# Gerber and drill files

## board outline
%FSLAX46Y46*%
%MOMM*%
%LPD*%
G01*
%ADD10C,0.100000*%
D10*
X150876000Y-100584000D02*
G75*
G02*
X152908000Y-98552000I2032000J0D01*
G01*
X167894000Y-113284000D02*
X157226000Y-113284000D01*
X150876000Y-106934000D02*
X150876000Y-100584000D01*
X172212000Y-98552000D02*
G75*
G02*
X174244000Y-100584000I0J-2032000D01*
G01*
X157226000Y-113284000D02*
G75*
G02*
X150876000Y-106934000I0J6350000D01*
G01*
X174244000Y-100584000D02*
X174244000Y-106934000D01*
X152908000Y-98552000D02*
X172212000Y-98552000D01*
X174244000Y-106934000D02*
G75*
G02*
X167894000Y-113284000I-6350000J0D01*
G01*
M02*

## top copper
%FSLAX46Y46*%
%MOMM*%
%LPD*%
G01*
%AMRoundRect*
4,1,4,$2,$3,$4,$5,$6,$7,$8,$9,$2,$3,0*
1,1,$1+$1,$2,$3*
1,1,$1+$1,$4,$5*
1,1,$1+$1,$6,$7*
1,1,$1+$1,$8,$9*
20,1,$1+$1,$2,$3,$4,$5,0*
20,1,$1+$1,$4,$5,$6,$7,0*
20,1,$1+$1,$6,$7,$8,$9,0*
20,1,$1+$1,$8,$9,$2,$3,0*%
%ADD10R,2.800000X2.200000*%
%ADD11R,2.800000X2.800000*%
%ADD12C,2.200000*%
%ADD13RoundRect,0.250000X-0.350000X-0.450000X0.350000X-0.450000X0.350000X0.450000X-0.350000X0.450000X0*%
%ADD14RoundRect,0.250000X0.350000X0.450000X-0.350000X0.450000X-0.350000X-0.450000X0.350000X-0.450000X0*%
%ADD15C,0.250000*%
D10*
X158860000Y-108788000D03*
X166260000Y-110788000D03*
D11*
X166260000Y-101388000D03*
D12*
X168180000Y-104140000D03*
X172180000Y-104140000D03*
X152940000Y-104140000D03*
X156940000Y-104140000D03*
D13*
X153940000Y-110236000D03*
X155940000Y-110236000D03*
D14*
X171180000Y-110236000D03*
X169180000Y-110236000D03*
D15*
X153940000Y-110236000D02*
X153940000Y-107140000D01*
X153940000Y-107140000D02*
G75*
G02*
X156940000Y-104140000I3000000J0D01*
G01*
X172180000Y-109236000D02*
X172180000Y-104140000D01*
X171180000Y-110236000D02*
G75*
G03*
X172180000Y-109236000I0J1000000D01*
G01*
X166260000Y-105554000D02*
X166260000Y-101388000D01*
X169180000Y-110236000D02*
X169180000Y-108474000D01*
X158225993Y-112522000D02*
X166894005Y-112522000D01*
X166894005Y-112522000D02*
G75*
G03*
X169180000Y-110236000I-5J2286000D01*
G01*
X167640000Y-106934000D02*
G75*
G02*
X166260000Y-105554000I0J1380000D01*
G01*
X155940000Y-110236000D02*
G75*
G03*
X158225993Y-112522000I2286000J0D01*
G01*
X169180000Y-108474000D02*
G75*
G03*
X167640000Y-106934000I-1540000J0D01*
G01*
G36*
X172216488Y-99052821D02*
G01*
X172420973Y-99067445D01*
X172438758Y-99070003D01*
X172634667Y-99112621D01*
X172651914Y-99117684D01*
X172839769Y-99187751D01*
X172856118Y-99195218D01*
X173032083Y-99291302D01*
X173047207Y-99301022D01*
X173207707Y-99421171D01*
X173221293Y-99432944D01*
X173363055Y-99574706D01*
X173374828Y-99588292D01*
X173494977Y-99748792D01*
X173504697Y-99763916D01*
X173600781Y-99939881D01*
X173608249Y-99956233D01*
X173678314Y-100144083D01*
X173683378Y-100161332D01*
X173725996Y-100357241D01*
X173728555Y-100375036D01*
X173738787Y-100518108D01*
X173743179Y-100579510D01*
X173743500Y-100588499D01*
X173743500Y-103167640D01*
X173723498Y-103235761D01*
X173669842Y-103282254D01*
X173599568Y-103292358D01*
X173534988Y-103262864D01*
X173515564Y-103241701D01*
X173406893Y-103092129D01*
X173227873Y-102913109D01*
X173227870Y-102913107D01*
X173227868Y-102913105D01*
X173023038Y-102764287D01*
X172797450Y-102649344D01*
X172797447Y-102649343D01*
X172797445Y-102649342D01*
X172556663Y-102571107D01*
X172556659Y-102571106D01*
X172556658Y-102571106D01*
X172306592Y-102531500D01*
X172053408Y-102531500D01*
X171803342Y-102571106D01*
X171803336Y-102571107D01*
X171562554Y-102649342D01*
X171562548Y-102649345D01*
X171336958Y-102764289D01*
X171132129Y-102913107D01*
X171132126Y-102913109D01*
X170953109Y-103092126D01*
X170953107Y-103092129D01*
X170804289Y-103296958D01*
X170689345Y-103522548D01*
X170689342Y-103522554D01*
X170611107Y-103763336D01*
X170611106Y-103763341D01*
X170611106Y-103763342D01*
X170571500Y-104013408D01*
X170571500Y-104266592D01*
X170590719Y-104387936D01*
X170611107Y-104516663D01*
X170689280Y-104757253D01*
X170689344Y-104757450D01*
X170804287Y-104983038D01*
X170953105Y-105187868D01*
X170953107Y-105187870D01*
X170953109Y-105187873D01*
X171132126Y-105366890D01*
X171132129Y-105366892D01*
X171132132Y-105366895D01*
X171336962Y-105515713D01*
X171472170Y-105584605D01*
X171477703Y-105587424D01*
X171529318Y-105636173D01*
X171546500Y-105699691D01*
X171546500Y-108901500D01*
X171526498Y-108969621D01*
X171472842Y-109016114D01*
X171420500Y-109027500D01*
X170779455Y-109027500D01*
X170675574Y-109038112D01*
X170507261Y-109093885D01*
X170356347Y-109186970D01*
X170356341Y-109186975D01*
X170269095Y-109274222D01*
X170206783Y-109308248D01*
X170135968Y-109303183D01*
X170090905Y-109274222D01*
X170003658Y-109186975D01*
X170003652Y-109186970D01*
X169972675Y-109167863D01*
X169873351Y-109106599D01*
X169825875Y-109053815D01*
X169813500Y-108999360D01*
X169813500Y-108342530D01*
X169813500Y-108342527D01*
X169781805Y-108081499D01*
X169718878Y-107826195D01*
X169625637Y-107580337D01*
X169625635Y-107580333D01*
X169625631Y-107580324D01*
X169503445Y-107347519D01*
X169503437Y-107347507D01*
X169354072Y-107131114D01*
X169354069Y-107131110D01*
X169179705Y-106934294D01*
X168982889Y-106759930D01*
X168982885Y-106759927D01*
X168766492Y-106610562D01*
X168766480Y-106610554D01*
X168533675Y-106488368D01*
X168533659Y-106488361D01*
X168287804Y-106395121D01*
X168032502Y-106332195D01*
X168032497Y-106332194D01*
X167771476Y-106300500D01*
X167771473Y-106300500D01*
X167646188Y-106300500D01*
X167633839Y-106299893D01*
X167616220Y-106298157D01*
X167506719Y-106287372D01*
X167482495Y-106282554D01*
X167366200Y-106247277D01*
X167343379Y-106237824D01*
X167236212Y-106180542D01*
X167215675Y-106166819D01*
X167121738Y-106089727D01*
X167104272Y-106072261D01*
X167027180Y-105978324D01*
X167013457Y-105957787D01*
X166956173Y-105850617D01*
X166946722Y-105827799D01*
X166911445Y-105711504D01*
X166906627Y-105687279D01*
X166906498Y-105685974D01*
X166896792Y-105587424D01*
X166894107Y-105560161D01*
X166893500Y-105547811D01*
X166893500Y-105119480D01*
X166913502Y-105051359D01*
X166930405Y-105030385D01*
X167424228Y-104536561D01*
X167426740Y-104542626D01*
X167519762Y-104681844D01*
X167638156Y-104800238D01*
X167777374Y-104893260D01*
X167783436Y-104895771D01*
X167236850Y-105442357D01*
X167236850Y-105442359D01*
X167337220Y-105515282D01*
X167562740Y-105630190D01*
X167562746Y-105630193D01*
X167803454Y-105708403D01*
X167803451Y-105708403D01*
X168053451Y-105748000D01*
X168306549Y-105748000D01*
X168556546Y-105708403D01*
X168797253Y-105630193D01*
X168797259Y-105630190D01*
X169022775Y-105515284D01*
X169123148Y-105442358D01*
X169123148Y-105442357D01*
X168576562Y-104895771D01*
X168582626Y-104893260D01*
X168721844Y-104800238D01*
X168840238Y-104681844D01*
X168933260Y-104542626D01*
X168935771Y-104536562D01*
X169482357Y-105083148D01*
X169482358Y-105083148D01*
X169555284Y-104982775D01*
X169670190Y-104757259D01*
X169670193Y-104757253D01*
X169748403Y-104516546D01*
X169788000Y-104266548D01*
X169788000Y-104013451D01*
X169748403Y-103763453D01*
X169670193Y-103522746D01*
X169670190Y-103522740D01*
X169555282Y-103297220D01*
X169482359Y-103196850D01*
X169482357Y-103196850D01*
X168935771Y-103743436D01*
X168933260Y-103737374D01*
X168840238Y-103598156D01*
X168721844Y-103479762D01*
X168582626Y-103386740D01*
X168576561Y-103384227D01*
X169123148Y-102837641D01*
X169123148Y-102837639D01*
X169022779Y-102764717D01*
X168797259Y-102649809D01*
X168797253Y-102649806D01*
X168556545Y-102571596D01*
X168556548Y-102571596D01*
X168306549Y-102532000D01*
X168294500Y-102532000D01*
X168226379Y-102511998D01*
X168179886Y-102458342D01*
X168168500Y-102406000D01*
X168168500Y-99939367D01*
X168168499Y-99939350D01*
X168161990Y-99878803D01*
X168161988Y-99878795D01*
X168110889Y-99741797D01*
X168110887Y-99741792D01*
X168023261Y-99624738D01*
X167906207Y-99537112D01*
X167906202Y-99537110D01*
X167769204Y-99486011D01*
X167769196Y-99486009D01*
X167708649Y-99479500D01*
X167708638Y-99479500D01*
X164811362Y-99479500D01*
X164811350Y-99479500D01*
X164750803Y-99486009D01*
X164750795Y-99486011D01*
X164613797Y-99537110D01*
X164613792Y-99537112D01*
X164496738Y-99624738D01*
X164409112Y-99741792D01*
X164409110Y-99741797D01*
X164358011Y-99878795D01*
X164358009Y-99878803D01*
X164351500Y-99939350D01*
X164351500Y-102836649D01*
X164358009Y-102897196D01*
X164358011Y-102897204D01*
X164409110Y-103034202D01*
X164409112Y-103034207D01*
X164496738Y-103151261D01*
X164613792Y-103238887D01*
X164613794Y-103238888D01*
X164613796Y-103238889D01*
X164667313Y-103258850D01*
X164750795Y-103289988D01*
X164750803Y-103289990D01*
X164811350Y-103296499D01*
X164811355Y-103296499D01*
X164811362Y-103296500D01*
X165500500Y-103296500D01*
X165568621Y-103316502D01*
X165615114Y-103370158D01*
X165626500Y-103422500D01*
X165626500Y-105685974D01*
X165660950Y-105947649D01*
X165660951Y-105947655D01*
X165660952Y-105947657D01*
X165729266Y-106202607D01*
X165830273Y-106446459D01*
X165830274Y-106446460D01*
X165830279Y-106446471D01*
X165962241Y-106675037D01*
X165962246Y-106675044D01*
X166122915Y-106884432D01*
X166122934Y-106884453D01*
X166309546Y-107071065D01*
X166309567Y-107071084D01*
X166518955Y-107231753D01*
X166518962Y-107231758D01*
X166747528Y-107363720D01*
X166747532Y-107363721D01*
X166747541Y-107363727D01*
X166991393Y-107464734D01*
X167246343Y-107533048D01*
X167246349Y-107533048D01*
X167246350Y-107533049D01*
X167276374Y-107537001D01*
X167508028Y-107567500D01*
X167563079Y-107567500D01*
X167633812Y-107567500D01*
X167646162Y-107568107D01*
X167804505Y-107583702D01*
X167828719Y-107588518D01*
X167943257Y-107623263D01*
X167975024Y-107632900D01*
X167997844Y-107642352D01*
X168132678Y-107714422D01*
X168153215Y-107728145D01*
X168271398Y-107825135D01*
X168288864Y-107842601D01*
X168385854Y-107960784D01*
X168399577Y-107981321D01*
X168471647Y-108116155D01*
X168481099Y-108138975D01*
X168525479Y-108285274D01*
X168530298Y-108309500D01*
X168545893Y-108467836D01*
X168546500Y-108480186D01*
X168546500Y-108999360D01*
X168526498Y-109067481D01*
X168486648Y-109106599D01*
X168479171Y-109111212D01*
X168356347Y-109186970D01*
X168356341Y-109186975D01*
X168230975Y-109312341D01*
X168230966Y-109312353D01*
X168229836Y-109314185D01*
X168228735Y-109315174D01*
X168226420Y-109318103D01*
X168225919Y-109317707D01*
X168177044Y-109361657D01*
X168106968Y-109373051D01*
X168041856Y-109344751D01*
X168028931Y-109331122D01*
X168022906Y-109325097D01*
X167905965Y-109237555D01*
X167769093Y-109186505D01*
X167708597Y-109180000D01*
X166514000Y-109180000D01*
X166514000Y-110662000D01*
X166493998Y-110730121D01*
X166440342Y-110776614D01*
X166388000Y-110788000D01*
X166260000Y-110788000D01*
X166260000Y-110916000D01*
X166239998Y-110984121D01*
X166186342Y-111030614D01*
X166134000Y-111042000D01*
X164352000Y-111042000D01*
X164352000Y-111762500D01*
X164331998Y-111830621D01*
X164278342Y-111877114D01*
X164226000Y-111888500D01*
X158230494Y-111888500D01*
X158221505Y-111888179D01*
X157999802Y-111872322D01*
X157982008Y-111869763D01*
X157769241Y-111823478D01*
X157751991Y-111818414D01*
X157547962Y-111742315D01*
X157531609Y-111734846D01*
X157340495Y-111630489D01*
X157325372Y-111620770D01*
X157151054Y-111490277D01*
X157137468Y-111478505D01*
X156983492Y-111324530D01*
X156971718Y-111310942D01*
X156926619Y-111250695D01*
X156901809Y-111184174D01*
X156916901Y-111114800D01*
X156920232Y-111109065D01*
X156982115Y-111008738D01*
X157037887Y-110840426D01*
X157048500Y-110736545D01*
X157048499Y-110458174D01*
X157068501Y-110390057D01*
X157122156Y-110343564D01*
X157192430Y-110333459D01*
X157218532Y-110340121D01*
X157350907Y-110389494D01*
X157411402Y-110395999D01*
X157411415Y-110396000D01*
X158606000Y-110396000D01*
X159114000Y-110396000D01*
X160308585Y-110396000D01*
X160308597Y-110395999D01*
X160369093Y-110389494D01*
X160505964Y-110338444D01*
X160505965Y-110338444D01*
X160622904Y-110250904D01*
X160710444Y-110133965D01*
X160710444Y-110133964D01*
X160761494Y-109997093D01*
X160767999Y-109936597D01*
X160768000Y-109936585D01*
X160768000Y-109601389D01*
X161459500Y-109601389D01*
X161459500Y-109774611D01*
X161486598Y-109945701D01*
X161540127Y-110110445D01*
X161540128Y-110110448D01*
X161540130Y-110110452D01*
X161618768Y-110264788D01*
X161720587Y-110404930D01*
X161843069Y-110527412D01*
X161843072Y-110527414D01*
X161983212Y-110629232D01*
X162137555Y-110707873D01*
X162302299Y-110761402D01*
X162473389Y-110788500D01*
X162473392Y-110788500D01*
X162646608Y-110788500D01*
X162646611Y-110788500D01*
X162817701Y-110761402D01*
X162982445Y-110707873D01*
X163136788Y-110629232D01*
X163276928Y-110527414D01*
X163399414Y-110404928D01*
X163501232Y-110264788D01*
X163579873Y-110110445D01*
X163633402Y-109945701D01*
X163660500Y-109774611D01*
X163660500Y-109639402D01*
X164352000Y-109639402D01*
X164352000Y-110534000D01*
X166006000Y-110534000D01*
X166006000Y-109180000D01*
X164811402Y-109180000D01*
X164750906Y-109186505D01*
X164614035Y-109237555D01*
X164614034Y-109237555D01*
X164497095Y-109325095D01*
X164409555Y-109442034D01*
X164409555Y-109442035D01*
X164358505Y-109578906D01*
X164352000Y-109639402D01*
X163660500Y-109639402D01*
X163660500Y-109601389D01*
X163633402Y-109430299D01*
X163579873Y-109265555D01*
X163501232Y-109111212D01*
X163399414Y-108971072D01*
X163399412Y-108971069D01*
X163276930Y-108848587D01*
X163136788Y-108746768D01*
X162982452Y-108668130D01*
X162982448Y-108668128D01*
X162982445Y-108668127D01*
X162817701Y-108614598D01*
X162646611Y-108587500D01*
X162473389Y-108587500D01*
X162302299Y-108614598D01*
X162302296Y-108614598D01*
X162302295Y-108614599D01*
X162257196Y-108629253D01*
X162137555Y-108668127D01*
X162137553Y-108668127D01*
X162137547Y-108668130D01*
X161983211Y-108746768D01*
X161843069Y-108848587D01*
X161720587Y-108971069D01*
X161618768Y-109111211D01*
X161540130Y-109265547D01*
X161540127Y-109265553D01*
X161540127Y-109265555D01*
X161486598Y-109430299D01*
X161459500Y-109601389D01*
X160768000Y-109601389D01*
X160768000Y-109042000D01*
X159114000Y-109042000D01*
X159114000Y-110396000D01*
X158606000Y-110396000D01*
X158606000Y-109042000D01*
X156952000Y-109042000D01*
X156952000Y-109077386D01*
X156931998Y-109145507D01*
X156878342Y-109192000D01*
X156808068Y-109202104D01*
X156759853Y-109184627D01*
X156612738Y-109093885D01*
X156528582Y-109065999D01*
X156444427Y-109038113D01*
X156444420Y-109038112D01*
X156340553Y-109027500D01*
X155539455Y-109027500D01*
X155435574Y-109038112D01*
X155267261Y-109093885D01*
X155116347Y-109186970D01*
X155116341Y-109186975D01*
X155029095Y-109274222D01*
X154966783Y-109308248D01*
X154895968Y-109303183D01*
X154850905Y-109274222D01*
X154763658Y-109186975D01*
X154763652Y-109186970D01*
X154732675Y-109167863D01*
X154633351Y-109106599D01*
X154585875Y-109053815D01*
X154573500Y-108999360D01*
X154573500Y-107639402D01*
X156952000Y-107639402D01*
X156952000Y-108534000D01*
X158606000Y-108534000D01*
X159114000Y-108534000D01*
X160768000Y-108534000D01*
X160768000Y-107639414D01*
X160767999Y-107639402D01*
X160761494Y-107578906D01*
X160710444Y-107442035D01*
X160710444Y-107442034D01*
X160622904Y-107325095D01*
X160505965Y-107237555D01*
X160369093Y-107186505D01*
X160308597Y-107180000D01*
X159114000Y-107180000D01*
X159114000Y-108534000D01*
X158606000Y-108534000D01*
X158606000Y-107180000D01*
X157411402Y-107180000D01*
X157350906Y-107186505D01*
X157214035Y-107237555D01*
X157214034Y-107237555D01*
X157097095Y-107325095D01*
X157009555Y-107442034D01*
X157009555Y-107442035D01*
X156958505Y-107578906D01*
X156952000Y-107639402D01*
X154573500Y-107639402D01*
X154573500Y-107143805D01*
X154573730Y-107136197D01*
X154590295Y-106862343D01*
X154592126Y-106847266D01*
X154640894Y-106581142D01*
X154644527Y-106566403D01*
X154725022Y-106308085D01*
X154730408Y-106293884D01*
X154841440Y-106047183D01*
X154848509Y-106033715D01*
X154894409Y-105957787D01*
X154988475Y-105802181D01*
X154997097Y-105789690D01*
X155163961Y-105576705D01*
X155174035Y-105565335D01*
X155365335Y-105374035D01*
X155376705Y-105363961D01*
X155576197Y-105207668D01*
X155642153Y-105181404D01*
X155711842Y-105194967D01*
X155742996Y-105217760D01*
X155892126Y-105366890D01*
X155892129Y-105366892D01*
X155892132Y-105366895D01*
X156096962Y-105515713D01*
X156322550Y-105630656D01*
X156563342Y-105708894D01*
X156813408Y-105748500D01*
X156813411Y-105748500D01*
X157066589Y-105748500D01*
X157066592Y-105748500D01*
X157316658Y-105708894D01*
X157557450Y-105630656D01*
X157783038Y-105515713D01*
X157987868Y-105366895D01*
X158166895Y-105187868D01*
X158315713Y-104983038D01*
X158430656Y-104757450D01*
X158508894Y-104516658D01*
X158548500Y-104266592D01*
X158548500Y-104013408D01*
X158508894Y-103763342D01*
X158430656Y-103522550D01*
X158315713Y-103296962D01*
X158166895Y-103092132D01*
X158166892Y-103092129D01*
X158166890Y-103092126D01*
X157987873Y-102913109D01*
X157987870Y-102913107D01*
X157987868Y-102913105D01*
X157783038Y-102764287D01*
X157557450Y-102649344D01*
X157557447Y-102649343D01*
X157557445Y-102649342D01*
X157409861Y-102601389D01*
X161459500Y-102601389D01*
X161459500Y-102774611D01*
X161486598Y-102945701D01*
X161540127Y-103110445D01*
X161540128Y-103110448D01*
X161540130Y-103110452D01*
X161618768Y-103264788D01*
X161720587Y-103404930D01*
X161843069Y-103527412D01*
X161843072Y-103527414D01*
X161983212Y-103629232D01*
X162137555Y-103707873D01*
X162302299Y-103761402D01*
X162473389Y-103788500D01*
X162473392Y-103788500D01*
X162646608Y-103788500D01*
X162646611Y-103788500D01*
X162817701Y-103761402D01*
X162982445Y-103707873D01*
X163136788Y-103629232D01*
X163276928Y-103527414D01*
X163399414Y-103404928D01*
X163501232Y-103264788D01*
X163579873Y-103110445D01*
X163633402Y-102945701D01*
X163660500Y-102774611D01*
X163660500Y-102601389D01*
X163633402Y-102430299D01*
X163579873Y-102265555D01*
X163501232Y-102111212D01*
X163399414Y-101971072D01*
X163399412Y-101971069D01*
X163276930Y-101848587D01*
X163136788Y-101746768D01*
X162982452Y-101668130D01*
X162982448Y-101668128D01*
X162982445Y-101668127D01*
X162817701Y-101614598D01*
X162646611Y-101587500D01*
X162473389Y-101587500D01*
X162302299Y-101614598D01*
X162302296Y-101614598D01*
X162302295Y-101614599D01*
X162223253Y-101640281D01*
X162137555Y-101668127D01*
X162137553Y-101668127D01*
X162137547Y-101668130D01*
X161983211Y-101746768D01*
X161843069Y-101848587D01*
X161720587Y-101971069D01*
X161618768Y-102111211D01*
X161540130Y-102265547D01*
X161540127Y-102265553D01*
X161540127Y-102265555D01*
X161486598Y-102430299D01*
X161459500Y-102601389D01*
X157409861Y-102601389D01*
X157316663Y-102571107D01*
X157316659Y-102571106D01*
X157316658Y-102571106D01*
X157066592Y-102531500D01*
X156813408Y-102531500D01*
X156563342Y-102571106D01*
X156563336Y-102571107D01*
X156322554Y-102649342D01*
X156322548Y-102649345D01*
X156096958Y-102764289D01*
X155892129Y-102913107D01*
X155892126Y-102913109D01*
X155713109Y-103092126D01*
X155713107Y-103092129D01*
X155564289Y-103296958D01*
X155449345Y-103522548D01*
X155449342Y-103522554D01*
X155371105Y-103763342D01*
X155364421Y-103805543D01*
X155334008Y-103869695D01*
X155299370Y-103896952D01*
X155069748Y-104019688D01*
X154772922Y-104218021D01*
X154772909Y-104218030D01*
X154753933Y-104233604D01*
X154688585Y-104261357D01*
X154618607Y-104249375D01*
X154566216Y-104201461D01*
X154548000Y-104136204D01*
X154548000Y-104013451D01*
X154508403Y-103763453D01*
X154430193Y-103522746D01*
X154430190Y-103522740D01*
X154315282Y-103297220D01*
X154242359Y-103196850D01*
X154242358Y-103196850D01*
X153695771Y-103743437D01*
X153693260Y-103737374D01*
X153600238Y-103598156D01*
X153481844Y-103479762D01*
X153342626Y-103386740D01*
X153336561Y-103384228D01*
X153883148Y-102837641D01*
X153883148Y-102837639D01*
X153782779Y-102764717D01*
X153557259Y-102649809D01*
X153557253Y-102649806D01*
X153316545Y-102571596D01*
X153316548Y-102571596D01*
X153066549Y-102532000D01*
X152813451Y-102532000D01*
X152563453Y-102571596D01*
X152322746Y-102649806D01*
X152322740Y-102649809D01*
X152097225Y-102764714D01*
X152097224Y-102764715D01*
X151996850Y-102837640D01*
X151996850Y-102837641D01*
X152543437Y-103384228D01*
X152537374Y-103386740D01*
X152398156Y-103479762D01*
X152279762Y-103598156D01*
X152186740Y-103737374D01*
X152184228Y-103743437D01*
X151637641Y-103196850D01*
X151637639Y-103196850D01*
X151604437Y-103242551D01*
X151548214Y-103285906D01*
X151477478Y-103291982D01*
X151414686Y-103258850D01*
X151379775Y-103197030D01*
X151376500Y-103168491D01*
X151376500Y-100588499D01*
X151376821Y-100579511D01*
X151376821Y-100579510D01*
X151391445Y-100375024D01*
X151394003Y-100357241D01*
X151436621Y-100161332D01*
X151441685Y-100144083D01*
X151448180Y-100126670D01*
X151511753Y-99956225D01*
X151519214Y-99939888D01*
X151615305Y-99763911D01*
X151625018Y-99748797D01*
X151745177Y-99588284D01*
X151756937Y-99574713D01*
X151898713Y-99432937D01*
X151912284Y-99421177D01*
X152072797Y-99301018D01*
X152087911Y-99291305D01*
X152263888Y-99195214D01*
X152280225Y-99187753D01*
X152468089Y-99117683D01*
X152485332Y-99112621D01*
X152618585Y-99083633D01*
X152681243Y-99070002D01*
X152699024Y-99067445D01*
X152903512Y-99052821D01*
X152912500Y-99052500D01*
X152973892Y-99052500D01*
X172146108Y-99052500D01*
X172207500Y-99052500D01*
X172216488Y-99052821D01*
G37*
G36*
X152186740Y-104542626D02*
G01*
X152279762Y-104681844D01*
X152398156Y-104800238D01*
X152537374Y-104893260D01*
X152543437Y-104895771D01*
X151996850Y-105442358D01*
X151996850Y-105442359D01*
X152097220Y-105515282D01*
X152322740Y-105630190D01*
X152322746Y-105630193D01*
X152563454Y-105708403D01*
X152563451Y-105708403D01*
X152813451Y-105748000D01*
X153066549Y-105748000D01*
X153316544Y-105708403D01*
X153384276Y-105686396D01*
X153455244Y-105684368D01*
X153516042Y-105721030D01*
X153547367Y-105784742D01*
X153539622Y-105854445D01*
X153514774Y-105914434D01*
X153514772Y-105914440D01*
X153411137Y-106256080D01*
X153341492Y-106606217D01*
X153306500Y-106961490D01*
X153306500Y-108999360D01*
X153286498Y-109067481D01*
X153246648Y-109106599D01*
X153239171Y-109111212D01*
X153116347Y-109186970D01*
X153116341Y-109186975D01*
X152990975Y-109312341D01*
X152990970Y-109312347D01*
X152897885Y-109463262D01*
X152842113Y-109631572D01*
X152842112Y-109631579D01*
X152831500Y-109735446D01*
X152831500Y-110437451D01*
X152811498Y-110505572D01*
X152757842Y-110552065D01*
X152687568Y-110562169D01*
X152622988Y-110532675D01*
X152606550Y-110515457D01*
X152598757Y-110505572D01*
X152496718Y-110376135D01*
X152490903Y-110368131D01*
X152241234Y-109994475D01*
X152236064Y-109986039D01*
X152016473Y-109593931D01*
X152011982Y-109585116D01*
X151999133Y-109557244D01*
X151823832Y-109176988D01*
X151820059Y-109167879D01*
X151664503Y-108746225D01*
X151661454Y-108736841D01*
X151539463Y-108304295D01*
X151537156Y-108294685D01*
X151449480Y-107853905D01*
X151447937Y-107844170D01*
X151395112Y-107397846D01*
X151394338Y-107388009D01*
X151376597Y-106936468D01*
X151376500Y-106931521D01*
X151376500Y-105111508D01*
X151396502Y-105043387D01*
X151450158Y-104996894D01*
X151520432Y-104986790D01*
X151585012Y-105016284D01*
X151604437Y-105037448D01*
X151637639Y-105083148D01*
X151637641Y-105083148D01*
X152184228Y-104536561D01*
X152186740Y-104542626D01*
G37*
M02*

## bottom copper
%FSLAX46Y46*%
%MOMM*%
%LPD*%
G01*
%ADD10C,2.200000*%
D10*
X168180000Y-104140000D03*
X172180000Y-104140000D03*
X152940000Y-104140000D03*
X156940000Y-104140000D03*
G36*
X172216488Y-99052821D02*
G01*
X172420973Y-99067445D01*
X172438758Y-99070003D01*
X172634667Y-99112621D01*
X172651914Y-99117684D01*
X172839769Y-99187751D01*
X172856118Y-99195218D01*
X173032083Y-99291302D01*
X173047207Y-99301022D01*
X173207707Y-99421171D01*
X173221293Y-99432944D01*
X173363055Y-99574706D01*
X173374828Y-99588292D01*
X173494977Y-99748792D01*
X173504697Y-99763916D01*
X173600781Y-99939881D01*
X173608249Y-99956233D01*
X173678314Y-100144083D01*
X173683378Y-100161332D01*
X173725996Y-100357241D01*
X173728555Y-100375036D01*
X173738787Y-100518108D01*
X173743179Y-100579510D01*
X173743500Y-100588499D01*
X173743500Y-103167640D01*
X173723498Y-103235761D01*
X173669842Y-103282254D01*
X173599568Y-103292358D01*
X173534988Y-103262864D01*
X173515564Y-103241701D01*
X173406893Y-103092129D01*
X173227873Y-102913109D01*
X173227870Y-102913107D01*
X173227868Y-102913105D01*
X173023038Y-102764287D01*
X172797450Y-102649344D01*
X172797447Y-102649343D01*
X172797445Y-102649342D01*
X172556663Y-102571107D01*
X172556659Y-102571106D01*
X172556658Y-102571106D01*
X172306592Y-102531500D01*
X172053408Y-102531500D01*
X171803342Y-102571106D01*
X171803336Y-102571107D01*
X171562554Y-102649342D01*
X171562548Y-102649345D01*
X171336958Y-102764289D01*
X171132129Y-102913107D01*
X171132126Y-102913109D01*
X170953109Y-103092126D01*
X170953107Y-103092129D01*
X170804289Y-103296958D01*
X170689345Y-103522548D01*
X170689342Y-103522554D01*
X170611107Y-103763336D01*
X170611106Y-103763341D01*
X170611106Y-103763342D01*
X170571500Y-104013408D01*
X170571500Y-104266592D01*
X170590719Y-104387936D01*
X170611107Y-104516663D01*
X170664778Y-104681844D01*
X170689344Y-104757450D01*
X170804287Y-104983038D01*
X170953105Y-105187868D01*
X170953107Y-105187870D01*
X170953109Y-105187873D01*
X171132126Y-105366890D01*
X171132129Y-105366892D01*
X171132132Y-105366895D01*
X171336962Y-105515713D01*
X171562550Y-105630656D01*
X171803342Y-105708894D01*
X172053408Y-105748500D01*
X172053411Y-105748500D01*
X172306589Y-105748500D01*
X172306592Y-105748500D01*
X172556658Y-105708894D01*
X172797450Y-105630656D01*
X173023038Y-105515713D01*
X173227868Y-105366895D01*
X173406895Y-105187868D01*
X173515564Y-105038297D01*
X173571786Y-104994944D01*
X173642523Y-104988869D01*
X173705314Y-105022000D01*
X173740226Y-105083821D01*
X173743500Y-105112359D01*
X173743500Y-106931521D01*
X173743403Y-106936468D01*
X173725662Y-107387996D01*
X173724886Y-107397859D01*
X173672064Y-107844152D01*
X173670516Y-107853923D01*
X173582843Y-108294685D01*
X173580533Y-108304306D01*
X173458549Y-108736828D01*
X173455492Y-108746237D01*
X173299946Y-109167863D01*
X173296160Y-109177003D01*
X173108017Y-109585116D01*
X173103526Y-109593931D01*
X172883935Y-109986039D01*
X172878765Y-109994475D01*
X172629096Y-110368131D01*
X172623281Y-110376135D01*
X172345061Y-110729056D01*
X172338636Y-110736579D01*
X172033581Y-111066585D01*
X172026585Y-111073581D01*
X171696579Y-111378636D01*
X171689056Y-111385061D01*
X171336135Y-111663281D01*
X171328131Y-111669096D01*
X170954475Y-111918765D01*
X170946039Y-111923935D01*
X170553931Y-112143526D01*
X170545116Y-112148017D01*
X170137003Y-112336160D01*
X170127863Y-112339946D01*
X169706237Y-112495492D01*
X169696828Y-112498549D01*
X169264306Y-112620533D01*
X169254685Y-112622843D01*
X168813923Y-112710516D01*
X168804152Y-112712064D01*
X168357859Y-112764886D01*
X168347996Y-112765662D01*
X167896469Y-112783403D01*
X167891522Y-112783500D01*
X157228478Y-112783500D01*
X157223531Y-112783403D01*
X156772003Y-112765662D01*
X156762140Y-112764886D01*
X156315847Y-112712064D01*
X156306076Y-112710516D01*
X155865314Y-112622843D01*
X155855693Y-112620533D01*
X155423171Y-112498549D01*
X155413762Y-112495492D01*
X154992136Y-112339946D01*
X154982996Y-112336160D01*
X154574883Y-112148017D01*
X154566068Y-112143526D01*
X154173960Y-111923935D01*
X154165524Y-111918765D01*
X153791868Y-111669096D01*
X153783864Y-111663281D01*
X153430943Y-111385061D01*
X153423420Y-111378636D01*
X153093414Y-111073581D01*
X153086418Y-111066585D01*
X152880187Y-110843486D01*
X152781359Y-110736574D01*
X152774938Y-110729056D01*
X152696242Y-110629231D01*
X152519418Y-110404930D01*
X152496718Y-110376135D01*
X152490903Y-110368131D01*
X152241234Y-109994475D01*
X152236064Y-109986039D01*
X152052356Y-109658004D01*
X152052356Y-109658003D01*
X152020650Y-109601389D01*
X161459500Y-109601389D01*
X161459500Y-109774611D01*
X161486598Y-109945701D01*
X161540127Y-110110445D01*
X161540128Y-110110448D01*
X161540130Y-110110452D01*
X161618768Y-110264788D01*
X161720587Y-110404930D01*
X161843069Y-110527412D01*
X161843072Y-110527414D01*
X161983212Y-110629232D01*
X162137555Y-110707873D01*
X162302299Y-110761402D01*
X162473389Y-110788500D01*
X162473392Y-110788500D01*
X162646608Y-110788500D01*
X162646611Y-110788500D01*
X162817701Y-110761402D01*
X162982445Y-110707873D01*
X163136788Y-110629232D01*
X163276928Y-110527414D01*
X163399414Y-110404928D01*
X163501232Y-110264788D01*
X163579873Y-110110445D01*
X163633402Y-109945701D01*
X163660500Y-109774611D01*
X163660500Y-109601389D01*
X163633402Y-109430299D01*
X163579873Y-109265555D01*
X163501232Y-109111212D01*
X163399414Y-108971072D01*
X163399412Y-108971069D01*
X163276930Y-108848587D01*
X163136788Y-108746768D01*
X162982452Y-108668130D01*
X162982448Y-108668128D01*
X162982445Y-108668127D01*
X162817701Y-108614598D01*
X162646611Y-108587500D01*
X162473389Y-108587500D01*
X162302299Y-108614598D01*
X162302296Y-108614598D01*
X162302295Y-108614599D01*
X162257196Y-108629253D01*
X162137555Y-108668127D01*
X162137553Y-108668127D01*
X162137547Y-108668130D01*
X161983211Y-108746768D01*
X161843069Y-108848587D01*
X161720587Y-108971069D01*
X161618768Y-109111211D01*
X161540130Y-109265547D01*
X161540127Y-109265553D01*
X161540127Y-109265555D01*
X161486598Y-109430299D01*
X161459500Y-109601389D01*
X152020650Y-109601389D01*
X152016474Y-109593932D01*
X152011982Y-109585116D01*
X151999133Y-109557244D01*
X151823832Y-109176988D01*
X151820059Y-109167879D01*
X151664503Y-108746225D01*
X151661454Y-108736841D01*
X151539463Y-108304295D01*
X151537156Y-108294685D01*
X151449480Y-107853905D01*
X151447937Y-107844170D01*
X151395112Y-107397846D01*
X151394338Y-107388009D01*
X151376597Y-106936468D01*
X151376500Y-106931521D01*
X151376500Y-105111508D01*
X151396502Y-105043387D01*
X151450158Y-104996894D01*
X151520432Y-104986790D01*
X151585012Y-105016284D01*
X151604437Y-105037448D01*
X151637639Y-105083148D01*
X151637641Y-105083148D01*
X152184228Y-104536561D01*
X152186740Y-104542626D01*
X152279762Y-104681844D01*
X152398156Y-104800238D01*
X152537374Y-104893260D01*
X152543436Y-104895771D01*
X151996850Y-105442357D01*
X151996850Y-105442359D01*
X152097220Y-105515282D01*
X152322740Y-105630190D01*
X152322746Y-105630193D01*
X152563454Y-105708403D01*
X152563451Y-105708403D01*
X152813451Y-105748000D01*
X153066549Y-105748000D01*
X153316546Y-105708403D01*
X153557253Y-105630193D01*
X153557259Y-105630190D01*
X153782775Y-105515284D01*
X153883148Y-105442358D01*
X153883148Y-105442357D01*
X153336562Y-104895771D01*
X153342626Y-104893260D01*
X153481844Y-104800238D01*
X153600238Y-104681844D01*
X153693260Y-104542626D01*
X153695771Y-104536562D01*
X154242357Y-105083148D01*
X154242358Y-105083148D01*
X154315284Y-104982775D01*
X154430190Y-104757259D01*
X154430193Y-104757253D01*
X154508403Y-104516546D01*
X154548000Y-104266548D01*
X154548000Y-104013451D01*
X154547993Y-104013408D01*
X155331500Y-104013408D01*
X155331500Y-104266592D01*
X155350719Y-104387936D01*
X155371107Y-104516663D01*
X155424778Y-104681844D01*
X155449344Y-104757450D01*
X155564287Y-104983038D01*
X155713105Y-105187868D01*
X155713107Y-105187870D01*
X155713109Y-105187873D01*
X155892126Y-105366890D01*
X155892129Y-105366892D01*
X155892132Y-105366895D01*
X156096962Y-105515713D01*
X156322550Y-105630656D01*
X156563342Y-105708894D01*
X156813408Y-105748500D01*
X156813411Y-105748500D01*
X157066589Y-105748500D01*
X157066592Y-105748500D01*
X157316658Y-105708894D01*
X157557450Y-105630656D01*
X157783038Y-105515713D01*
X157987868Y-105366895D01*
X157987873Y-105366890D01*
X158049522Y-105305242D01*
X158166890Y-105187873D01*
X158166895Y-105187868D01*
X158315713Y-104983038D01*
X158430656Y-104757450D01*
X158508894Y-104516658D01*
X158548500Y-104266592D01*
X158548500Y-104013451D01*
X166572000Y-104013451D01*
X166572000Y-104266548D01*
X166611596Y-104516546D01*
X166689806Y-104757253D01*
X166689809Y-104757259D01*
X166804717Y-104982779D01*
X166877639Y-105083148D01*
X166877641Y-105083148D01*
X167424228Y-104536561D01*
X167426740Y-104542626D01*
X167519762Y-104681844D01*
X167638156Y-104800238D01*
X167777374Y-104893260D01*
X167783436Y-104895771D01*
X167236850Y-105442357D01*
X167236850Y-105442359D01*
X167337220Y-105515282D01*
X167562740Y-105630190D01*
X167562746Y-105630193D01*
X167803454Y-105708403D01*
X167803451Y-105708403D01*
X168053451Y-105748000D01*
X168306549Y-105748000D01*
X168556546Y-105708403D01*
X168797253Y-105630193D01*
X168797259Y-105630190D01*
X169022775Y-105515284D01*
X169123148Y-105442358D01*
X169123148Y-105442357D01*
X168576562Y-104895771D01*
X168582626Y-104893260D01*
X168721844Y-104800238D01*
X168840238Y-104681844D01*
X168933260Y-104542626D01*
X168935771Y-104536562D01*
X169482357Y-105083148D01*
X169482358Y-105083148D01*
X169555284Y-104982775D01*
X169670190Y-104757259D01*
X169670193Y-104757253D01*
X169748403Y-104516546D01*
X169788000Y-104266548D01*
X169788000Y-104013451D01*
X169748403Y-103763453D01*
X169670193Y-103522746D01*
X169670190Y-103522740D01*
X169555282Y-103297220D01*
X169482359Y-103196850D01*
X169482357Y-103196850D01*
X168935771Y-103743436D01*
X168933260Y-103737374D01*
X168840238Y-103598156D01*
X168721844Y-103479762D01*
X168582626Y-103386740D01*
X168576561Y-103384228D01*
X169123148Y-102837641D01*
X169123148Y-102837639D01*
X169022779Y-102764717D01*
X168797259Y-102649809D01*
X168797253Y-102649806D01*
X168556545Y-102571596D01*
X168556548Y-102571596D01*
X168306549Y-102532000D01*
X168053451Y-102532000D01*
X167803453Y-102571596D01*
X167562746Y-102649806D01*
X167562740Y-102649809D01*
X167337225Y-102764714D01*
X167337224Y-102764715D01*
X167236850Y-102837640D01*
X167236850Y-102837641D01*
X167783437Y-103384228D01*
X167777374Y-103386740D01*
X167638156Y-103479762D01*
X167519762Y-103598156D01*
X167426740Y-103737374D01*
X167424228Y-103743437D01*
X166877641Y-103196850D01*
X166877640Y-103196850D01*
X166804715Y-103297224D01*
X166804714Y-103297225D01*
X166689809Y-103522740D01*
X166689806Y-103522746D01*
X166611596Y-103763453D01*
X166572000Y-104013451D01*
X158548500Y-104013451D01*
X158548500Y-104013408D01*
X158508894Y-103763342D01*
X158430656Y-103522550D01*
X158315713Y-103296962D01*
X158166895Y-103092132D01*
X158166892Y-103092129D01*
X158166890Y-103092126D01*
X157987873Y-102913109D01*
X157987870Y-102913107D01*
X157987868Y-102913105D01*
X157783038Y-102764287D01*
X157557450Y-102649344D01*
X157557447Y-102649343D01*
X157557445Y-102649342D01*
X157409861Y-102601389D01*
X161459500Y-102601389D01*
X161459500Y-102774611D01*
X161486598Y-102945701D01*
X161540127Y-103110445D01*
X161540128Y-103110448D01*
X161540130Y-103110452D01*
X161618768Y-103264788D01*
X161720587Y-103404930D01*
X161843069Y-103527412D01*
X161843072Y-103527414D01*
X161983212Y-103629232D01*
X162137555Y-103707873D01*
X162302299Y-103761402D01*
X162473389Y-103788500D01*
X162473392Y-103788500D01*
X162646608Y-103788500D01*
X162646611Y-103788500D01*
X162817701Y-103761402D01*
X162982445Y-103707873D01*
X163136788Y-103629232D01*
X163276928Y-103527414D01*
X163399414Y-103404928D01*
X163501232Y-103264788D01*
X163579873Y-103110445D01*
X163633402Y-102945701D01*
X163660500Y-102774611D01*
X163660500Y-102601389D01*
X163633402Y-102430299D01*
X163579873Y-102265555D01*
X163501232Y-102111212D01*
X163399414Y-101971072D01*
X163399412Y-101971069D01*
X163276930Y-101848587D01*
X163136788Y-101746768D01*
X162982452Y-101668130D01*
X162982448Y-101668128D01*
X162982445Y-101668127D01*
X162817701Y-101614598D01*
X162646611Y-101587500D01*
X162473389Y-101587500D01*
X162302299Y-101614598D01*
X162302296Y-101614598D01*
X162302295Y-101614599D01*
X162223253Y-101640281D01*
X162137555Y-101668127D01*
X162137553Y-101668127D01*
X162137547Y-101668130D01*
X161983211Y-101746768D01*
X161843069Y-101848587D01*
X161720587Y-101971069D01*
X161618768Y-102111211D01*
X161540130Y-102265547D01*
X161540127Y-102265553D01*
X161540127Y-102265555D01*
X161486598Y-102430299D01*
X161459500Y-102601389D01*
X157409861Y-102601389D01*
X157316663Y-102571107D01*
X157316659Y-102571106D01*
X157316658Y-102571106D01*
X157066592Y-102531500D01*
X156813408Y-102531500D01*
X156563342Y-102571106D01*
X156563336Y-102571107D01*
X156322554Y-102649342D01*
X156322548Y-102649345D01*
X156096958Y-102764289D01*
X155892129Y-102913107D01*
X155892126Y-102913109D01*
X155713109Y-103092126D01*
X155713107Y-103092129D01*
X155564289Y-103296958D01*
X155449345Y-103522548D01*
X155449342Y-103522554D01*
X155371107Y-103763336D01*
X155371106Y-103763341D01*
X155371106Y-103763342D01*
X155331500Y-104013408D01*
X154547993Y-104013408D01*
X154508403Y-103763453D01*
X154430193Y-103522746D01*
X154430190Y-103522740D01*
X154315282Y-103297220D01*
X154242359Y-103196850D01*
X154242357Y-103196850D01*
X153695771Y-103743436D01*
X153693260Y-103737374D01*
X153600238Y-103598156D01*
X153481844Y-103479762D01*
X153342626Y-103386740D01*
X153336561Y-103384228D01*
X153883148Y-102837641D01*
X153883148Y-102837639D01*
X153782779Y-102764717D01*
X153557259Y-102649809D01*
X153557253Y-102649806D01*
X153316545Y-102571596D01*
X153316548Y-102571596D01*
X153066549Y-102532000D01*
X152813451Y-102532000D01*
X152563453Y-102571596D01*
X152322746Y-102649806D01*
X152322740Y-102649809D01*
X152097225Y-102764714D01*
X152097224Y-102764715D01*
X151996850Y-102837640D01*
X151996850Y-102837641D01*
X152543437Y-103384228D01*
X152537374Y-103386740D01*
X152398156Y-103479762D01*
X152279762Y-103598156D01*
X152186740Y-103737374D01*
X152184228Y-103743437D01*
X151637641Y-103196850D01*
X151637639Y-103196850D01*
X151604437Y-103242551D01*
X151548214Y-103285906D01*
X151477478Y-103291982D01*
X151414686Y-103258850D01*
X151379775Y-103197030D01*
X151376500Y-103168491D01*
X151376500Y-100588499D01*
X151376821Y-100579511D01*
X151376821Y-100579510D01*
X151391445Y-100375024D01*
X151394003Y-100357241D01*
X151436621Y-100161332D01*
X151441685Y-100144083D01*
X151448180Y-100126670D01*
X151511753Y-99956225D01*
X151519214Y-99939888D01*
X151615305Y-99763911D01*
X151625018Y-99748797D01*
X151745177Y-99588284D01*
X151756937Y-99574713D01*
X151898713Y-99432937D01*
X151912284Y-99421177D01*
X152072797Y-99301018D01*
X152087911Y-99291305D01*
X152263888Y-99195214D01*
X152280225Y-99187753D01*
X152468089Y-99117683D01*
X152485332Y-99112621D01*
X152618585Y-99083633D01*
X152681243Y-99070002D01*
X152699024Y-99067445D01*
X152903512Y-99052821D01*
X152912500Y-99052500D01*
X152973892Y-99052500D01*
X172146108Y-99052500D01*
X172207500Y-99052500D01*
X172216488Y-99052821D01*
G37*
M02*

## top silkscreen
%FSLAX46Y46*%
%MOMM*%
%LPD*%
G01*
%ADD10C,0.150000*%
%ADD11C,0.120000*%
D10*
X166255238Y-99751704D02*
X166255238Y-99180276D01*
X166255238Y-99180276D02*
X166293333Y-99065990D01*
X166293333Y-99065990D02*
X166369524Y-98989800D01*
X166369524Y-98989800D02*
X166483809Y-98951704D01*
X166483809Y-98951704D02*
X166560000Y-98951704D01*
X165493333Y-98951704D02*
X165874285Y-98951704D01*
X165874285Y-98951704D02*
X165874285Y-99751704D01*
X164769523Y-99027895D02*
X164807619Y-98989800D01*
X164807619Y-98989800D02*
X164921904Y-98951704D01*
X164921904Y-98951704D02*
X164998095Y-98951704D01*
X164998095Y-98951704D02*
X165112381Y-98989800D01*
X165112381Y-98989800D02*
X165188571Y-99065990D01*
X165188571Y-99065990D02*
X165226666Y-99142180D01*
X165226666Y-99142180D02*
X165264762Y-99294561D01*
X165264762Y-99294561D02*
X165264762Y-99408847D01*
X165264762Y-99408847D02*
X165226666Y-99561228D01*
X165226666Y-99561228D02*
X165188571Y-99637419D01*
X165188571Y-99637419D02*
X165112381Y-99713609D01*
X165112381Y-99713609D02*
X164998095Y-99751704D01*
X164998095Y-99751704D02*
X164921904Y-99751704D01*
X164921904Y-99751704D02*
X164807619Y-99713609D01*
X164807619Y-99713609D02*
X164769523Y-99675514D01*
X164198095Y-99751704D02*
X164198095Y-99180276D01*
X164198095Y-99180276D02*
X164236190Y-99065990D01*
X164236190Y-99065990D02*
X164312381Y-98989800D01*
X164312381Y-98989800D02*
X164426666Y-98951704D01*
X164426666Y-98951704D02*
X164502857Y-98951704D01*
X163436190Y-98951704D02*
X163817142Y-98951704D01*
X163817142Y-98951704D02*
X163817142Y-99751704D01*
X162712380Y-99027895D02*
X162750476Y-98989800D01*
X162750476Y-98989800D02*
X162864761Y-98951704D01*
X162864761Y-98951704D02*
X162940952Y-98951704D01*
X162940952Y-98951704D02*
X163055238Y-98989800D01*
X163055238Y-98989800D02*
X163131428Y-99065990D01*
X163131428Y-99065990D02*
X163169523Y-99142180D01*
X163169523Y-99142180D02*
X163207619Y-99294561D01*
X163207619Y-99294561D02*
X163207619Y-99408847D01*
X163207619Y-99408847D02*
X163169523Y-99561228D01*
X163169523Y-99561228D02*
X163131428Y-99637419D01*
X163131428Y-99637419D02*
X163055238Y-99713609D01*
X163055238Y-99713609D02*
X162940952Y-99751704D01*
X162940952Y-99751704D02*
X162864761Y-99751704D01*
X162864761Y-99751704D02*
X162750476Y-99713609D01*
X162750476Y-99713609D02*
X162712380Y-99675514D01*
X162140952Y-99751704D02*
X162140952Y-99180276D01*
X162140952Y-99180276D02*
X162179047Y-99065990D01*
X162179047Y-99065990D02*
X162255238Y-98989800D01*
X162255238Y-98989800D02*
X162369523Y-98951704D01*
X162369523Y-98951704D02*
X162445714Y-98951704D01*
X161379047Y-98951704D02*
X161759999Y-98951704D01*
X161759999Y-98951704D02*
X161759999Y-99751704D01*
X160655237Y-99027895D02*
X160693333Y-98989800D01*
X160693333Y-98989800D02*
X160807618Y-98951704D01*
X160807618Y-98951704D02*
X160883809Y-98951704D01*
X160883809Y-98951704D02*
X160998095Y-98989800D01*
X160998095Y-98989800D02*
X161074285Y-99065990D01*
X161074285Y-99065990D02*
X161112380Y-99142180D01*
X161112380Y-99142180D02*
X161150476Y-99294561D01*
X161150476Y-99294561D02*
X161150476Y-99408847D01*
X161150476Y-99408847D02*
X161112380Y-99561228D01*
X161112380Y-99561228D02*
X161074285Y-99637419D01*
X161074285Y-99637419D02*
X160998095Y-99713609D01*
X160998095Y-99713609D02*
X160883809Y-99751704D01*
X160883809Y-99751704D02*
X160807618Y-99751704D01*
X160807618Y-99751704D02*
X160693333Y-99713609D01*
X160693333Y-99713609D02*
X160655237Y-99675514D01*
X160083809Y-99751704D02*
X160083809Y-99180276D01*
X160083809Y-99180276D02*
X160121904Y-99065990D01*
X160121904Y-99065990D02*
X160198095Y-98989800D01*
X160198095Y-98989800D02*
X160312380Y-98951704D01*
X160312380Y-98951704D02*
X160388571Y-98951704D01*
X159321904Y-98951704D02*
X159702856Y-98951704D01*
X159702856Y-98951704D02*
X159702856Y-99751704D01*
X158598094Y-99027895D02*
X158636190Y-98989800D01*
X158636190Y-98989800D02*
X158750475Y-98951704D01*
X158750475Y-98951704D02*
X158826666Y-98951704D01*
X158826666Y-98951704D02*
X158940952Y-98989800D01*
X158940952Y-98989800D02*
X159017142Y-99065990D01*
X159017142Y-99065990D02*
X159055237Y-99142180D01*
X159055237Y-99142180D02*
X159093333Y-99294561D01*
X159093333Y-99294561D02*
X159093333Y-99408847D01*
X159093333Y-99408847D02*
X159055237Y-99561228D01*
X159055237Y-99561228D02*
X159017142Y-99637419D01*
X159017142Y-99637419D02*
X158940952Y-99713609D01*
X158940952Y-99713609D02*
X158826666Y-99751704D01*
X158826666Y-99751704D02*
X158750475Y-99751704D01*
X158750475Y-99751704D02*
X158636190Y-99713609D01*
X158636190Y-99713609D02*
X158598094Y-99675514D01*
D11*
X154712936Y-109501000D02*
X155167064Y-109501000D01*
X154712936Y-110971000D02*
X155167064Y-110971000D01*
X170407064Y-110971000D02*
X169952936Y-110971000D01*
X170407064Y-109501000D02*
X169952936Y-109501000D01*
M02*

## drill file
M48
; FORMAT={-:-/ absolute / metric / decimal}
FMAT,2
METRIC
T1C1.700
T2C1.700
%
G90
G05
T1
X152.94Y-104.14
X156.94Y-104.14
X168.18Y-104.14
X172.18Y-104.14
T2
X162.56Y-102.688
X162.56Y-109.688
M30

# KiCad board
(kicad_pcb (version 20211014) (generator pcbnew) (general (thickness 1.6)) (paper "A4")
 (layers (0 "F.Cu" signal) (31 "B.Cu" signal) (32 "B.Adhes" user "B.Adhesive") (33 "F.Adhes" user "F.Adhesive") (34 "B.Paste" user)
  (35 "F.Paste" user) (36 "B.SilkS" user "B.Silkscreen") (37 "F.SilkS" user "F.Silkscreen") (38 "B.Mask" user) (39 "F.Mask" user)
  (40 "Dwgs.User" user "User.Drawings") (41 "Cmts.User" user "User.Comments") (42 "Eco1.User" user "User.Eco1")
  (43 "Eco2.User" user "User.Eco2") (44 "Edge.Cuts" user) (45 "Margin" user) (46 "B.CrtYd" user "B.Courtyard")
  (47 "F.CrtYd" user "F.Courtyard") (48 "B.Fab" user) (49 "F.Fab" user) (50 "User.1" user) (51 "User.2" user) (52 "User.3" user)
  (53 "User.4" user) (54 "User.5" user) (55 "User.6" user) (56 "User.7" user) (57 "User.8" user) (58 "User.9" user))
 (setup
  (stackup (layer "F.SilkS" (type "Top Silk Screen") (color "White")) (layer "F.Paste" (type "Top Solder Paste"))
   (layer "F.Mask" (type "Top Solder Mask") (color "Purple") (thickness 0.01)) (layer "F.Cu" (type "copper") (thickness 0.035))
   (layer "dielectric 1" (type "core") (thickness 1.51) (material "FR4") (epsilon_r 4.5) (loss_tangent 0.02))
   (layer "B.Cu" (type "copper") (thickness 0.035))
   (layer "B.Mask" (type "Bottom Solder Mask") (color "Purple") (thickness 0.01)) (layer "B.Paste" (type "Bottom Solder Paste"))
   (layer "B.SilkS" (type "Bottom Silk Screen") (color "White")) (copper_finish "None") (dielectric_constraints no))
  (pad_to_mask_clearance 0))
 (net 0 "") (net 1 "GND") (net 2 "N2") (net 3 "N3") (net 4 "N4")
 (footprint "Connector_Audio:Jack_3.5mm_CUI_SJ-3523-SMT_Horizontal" (layer "F.Cu") (at 162.56 107.188 180)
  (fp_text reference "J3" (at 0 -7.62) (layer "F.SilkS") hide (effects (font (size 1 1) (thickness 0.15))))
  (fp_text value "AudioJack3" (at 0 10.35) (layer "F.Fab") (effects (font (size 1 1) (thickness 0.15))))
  (pad "" np_thru_hole circle (at 0 4.5 180) (size 1.7 1.7) (drill 1.7) (layers *.Cu *.Mask))
  (pad "" np_thru_hole circle (at 0 -2.5 180) (size 1.7 1.7) (drill 1.7) (layers *.Cu *.Mask))
  (pad "R" smd rect (at 3.7 -1.6 180) (size 2.8 2.2) (layers "F.Cu" "F.Paste" "F.Mask") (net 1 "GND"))
  (pad "S" smd rect (at -3.7 -3.6 180) (size 2.8 2.2) (layers "F.Cu" "F.Paste" "F.Mask") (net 1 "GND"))
  (pad "T" smd rect (at -3.7 5.8 180) (size 2.8 2.8) (layers "F.Cu" "F.Paste" "F.Mask") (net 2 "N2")))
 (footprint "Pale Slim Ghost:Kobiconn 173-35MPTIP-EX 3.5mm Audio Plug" (layer "F.Cu") (at 170.18 104.14)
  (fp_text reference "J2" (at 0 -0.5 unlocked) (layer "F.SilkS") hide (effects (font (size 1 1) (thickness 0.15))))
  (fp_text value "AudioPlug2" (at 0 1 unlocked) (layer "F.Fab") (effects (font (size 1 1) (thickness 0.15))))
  (pad "S" thru_hole circle (at -2 0) (size 2.2 2.2) (drill 1.7) (layers *.Cu *.Mask) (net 1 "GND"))
  (pad "T" thru_hole circle (at 2 0) (size 2.2 2.2) (drill 1.7) (layers *.Cu *.Mask) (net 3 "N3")))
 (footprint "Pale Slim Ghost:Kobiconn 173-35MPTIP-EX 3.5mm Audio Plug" (layer "F.Cu") (at 154.94 104.14)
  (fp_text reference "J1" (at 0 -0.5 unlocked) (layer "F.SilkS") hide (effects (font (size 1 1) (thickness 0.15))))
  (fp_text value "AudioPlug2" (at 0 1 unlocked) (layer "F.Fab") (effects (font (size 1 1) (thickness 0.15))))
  (pad "S" thru_hole circle (at -2 0) (size 2.2 2.2) (drill 1.7) (layers *.Cu *.Mask) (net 1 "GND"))
  (pad "T" thru_hole circle (at 2 0) (size 2.2 2.2) (drill 1.7) (layers *.Cu *.Mask) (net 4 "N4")))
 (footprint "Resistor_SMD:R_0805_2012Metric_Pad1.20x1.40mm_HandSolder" (layer "F.Cu") (at 154.94 110.236)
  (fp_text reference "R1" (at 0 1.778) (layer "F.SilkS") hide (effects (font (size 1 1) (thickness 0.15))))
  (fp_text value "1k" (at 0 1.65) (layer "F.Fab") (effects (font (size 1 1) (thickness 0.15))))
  (fp_line (start -0.227064 -0.735) (end 0.227064 -0.735) (layer "F.SilkS") (width 0.12))
  (fp_line (start -0.227064 0.735) (end 0.227064 0.735) (layer "F.SilkS") (width 0.12))
  (pad "1" smd roundrect (at -1 0) (size 1.2 1.4) (layers "F.Cu" "F.Paste" "F.Mask") (roundrect_rratio 0.208333) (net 4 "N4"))
  (pad "2" smd roundrect (at 1 0) (size 1.2 1.4) (layers "F.Cu" "F.Paste" "F.Mask") (roundrect_rratio 0.208333) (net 2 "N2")))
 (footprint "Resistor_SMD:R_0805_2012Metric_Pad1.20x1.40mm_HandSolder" (layer "F.Cu") (at 170.18 110.236 180)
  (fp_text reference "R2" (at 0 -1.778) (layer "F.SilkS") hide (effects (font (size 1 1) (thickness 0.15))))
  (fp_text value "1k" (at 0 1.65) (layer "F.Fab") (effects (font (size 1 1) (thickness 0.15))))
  (fp_line (start -0.227064 -0.735) (end 0.227064 -0.735) (layer "F.SilkS") (width 0.12))
  (fp_line (start -0.227064 0.735) (end 0.227064 0.735) (layer "F.SilkS") (width 0.12))
  (pad "1" smd roundrect (at -1 0 180) (size 1.2 1.4) (layers "F.Cu" "F.Paste" "F.Mask") (roundrect_rratio 0.208333) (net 3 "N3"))
  (pad "2" smd roundrect (at 1 0 180) (size 1.2 1.4) (layers "F.Cu" "F.Paste" "F.Mask") (roundrect_rratio 0.208333) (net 2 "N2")))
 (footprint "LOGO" (layer "B.Cu") (at 162.810681 106.033208)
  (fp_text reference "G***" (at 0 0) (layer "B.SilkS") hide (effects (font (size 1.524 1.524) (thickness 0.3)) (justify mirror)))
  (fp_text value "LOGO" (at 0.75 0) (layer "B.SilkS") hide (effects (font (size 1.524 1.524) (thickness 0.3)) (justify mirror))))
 (gr_arc (start 150.876 100.584) (mid 151.471159 99.147159) (end 152.908 98.552) (layer "Edge.Cuts") (width 0.1))
 (gr_line (start 167.894 113.284) (end 157.226 113.284) (layer "Edge.Cuts") (width 0.1))
 (gr_line (start 150.876 106.934) (end 150.876 100.584) (layer "Edge.Cuts") (width 0.1))
 (gr_arc (start 172.212 98.552) (mid 173.648841 99.147159) (end 174.244 100.584) (layer "Edge.Cuts") (width 0.1))
 (gr_arc (start 157.226 113.284) (mid 152.735872 111.424128) (end 150.876 106.934) (layer "Edge.Cuts") (width 0.1))
 (gr_line (start 174.244 100.584) (end 174.244 106.934) (layer "Edge.Cuts") (width 0.1))
 (gr_line (start 152.908 98.552) (end 172.212 98.552) (layer "Edge.Cuts") (width 0.1))
 (gr_arc (start 174.244 106.934) (mid 172.384128 111.424128) (end 167.894 113.284) (layer "Edge.Cuts") (width 0.1))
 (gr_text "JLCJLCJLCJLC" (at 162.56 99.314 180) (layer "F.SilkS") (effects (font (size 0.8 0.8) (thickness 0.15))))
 (segment (start 153.94 110.236) (end 153.94 107.14) (width 0.25) (layer "F.Cu") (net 4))
 (arc (start 153.94 107.14) (mid 154.81868 105.01868) (end 156.94 104.14) (width 0.25) (layer "F.Cu") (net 4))
 (segment (start 172.18 109.236) (end 172.18 104.14) (width 0.25) (layer "F.Cu") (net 3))
 (arc (start 171.18 110.236) (mid 171.887107 109.943107) (end 172.18 109.236) (width 0.25) (layer "F.Cu") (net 3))
 (segment (start 166.26 105.554) (end 166.26 101.388) (width 0.25) (layer "F.Cu") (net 2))
 (segment (start 169.18 110.236) (end 169.18 108.474) (width 0.25) (layer "F.Cu") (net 2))
 (segment (start 158.225993 112.522) (end 166.894005 112.522) (width 0.25) (layer "F.Cu") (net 2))
 (arc (start 166.894005 112.522) (mid 168.510448 111.852448) (end 169.18 110.236) (width 0.25) (layer "F.Cu") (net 2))
 (arc (start 167.64 106.934) (mid 166.664193 106.529807) (end 166.26 105.554) (width 0.25) (layer "F.Cu") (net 2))
 (arc (start 155.94 110.236) (mid 156.609552 111.852448) (end 158.225993 112.522) (width 0.25) (layer "F.Cu") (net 2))
 (arc (start 169.18 108.474) (mid 168.728944 107.385056) (end 167.64 106.934) (width 0.25) (layer "F.Cu") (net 2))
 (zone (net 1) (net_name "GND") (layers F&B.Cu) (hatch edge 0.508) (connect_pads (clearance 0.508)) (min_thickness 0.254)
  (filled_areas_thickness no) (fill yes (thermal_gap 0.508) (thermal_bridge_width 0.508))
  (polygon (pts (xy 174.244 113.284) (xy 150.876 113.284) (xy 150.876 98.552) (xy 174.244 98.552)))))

